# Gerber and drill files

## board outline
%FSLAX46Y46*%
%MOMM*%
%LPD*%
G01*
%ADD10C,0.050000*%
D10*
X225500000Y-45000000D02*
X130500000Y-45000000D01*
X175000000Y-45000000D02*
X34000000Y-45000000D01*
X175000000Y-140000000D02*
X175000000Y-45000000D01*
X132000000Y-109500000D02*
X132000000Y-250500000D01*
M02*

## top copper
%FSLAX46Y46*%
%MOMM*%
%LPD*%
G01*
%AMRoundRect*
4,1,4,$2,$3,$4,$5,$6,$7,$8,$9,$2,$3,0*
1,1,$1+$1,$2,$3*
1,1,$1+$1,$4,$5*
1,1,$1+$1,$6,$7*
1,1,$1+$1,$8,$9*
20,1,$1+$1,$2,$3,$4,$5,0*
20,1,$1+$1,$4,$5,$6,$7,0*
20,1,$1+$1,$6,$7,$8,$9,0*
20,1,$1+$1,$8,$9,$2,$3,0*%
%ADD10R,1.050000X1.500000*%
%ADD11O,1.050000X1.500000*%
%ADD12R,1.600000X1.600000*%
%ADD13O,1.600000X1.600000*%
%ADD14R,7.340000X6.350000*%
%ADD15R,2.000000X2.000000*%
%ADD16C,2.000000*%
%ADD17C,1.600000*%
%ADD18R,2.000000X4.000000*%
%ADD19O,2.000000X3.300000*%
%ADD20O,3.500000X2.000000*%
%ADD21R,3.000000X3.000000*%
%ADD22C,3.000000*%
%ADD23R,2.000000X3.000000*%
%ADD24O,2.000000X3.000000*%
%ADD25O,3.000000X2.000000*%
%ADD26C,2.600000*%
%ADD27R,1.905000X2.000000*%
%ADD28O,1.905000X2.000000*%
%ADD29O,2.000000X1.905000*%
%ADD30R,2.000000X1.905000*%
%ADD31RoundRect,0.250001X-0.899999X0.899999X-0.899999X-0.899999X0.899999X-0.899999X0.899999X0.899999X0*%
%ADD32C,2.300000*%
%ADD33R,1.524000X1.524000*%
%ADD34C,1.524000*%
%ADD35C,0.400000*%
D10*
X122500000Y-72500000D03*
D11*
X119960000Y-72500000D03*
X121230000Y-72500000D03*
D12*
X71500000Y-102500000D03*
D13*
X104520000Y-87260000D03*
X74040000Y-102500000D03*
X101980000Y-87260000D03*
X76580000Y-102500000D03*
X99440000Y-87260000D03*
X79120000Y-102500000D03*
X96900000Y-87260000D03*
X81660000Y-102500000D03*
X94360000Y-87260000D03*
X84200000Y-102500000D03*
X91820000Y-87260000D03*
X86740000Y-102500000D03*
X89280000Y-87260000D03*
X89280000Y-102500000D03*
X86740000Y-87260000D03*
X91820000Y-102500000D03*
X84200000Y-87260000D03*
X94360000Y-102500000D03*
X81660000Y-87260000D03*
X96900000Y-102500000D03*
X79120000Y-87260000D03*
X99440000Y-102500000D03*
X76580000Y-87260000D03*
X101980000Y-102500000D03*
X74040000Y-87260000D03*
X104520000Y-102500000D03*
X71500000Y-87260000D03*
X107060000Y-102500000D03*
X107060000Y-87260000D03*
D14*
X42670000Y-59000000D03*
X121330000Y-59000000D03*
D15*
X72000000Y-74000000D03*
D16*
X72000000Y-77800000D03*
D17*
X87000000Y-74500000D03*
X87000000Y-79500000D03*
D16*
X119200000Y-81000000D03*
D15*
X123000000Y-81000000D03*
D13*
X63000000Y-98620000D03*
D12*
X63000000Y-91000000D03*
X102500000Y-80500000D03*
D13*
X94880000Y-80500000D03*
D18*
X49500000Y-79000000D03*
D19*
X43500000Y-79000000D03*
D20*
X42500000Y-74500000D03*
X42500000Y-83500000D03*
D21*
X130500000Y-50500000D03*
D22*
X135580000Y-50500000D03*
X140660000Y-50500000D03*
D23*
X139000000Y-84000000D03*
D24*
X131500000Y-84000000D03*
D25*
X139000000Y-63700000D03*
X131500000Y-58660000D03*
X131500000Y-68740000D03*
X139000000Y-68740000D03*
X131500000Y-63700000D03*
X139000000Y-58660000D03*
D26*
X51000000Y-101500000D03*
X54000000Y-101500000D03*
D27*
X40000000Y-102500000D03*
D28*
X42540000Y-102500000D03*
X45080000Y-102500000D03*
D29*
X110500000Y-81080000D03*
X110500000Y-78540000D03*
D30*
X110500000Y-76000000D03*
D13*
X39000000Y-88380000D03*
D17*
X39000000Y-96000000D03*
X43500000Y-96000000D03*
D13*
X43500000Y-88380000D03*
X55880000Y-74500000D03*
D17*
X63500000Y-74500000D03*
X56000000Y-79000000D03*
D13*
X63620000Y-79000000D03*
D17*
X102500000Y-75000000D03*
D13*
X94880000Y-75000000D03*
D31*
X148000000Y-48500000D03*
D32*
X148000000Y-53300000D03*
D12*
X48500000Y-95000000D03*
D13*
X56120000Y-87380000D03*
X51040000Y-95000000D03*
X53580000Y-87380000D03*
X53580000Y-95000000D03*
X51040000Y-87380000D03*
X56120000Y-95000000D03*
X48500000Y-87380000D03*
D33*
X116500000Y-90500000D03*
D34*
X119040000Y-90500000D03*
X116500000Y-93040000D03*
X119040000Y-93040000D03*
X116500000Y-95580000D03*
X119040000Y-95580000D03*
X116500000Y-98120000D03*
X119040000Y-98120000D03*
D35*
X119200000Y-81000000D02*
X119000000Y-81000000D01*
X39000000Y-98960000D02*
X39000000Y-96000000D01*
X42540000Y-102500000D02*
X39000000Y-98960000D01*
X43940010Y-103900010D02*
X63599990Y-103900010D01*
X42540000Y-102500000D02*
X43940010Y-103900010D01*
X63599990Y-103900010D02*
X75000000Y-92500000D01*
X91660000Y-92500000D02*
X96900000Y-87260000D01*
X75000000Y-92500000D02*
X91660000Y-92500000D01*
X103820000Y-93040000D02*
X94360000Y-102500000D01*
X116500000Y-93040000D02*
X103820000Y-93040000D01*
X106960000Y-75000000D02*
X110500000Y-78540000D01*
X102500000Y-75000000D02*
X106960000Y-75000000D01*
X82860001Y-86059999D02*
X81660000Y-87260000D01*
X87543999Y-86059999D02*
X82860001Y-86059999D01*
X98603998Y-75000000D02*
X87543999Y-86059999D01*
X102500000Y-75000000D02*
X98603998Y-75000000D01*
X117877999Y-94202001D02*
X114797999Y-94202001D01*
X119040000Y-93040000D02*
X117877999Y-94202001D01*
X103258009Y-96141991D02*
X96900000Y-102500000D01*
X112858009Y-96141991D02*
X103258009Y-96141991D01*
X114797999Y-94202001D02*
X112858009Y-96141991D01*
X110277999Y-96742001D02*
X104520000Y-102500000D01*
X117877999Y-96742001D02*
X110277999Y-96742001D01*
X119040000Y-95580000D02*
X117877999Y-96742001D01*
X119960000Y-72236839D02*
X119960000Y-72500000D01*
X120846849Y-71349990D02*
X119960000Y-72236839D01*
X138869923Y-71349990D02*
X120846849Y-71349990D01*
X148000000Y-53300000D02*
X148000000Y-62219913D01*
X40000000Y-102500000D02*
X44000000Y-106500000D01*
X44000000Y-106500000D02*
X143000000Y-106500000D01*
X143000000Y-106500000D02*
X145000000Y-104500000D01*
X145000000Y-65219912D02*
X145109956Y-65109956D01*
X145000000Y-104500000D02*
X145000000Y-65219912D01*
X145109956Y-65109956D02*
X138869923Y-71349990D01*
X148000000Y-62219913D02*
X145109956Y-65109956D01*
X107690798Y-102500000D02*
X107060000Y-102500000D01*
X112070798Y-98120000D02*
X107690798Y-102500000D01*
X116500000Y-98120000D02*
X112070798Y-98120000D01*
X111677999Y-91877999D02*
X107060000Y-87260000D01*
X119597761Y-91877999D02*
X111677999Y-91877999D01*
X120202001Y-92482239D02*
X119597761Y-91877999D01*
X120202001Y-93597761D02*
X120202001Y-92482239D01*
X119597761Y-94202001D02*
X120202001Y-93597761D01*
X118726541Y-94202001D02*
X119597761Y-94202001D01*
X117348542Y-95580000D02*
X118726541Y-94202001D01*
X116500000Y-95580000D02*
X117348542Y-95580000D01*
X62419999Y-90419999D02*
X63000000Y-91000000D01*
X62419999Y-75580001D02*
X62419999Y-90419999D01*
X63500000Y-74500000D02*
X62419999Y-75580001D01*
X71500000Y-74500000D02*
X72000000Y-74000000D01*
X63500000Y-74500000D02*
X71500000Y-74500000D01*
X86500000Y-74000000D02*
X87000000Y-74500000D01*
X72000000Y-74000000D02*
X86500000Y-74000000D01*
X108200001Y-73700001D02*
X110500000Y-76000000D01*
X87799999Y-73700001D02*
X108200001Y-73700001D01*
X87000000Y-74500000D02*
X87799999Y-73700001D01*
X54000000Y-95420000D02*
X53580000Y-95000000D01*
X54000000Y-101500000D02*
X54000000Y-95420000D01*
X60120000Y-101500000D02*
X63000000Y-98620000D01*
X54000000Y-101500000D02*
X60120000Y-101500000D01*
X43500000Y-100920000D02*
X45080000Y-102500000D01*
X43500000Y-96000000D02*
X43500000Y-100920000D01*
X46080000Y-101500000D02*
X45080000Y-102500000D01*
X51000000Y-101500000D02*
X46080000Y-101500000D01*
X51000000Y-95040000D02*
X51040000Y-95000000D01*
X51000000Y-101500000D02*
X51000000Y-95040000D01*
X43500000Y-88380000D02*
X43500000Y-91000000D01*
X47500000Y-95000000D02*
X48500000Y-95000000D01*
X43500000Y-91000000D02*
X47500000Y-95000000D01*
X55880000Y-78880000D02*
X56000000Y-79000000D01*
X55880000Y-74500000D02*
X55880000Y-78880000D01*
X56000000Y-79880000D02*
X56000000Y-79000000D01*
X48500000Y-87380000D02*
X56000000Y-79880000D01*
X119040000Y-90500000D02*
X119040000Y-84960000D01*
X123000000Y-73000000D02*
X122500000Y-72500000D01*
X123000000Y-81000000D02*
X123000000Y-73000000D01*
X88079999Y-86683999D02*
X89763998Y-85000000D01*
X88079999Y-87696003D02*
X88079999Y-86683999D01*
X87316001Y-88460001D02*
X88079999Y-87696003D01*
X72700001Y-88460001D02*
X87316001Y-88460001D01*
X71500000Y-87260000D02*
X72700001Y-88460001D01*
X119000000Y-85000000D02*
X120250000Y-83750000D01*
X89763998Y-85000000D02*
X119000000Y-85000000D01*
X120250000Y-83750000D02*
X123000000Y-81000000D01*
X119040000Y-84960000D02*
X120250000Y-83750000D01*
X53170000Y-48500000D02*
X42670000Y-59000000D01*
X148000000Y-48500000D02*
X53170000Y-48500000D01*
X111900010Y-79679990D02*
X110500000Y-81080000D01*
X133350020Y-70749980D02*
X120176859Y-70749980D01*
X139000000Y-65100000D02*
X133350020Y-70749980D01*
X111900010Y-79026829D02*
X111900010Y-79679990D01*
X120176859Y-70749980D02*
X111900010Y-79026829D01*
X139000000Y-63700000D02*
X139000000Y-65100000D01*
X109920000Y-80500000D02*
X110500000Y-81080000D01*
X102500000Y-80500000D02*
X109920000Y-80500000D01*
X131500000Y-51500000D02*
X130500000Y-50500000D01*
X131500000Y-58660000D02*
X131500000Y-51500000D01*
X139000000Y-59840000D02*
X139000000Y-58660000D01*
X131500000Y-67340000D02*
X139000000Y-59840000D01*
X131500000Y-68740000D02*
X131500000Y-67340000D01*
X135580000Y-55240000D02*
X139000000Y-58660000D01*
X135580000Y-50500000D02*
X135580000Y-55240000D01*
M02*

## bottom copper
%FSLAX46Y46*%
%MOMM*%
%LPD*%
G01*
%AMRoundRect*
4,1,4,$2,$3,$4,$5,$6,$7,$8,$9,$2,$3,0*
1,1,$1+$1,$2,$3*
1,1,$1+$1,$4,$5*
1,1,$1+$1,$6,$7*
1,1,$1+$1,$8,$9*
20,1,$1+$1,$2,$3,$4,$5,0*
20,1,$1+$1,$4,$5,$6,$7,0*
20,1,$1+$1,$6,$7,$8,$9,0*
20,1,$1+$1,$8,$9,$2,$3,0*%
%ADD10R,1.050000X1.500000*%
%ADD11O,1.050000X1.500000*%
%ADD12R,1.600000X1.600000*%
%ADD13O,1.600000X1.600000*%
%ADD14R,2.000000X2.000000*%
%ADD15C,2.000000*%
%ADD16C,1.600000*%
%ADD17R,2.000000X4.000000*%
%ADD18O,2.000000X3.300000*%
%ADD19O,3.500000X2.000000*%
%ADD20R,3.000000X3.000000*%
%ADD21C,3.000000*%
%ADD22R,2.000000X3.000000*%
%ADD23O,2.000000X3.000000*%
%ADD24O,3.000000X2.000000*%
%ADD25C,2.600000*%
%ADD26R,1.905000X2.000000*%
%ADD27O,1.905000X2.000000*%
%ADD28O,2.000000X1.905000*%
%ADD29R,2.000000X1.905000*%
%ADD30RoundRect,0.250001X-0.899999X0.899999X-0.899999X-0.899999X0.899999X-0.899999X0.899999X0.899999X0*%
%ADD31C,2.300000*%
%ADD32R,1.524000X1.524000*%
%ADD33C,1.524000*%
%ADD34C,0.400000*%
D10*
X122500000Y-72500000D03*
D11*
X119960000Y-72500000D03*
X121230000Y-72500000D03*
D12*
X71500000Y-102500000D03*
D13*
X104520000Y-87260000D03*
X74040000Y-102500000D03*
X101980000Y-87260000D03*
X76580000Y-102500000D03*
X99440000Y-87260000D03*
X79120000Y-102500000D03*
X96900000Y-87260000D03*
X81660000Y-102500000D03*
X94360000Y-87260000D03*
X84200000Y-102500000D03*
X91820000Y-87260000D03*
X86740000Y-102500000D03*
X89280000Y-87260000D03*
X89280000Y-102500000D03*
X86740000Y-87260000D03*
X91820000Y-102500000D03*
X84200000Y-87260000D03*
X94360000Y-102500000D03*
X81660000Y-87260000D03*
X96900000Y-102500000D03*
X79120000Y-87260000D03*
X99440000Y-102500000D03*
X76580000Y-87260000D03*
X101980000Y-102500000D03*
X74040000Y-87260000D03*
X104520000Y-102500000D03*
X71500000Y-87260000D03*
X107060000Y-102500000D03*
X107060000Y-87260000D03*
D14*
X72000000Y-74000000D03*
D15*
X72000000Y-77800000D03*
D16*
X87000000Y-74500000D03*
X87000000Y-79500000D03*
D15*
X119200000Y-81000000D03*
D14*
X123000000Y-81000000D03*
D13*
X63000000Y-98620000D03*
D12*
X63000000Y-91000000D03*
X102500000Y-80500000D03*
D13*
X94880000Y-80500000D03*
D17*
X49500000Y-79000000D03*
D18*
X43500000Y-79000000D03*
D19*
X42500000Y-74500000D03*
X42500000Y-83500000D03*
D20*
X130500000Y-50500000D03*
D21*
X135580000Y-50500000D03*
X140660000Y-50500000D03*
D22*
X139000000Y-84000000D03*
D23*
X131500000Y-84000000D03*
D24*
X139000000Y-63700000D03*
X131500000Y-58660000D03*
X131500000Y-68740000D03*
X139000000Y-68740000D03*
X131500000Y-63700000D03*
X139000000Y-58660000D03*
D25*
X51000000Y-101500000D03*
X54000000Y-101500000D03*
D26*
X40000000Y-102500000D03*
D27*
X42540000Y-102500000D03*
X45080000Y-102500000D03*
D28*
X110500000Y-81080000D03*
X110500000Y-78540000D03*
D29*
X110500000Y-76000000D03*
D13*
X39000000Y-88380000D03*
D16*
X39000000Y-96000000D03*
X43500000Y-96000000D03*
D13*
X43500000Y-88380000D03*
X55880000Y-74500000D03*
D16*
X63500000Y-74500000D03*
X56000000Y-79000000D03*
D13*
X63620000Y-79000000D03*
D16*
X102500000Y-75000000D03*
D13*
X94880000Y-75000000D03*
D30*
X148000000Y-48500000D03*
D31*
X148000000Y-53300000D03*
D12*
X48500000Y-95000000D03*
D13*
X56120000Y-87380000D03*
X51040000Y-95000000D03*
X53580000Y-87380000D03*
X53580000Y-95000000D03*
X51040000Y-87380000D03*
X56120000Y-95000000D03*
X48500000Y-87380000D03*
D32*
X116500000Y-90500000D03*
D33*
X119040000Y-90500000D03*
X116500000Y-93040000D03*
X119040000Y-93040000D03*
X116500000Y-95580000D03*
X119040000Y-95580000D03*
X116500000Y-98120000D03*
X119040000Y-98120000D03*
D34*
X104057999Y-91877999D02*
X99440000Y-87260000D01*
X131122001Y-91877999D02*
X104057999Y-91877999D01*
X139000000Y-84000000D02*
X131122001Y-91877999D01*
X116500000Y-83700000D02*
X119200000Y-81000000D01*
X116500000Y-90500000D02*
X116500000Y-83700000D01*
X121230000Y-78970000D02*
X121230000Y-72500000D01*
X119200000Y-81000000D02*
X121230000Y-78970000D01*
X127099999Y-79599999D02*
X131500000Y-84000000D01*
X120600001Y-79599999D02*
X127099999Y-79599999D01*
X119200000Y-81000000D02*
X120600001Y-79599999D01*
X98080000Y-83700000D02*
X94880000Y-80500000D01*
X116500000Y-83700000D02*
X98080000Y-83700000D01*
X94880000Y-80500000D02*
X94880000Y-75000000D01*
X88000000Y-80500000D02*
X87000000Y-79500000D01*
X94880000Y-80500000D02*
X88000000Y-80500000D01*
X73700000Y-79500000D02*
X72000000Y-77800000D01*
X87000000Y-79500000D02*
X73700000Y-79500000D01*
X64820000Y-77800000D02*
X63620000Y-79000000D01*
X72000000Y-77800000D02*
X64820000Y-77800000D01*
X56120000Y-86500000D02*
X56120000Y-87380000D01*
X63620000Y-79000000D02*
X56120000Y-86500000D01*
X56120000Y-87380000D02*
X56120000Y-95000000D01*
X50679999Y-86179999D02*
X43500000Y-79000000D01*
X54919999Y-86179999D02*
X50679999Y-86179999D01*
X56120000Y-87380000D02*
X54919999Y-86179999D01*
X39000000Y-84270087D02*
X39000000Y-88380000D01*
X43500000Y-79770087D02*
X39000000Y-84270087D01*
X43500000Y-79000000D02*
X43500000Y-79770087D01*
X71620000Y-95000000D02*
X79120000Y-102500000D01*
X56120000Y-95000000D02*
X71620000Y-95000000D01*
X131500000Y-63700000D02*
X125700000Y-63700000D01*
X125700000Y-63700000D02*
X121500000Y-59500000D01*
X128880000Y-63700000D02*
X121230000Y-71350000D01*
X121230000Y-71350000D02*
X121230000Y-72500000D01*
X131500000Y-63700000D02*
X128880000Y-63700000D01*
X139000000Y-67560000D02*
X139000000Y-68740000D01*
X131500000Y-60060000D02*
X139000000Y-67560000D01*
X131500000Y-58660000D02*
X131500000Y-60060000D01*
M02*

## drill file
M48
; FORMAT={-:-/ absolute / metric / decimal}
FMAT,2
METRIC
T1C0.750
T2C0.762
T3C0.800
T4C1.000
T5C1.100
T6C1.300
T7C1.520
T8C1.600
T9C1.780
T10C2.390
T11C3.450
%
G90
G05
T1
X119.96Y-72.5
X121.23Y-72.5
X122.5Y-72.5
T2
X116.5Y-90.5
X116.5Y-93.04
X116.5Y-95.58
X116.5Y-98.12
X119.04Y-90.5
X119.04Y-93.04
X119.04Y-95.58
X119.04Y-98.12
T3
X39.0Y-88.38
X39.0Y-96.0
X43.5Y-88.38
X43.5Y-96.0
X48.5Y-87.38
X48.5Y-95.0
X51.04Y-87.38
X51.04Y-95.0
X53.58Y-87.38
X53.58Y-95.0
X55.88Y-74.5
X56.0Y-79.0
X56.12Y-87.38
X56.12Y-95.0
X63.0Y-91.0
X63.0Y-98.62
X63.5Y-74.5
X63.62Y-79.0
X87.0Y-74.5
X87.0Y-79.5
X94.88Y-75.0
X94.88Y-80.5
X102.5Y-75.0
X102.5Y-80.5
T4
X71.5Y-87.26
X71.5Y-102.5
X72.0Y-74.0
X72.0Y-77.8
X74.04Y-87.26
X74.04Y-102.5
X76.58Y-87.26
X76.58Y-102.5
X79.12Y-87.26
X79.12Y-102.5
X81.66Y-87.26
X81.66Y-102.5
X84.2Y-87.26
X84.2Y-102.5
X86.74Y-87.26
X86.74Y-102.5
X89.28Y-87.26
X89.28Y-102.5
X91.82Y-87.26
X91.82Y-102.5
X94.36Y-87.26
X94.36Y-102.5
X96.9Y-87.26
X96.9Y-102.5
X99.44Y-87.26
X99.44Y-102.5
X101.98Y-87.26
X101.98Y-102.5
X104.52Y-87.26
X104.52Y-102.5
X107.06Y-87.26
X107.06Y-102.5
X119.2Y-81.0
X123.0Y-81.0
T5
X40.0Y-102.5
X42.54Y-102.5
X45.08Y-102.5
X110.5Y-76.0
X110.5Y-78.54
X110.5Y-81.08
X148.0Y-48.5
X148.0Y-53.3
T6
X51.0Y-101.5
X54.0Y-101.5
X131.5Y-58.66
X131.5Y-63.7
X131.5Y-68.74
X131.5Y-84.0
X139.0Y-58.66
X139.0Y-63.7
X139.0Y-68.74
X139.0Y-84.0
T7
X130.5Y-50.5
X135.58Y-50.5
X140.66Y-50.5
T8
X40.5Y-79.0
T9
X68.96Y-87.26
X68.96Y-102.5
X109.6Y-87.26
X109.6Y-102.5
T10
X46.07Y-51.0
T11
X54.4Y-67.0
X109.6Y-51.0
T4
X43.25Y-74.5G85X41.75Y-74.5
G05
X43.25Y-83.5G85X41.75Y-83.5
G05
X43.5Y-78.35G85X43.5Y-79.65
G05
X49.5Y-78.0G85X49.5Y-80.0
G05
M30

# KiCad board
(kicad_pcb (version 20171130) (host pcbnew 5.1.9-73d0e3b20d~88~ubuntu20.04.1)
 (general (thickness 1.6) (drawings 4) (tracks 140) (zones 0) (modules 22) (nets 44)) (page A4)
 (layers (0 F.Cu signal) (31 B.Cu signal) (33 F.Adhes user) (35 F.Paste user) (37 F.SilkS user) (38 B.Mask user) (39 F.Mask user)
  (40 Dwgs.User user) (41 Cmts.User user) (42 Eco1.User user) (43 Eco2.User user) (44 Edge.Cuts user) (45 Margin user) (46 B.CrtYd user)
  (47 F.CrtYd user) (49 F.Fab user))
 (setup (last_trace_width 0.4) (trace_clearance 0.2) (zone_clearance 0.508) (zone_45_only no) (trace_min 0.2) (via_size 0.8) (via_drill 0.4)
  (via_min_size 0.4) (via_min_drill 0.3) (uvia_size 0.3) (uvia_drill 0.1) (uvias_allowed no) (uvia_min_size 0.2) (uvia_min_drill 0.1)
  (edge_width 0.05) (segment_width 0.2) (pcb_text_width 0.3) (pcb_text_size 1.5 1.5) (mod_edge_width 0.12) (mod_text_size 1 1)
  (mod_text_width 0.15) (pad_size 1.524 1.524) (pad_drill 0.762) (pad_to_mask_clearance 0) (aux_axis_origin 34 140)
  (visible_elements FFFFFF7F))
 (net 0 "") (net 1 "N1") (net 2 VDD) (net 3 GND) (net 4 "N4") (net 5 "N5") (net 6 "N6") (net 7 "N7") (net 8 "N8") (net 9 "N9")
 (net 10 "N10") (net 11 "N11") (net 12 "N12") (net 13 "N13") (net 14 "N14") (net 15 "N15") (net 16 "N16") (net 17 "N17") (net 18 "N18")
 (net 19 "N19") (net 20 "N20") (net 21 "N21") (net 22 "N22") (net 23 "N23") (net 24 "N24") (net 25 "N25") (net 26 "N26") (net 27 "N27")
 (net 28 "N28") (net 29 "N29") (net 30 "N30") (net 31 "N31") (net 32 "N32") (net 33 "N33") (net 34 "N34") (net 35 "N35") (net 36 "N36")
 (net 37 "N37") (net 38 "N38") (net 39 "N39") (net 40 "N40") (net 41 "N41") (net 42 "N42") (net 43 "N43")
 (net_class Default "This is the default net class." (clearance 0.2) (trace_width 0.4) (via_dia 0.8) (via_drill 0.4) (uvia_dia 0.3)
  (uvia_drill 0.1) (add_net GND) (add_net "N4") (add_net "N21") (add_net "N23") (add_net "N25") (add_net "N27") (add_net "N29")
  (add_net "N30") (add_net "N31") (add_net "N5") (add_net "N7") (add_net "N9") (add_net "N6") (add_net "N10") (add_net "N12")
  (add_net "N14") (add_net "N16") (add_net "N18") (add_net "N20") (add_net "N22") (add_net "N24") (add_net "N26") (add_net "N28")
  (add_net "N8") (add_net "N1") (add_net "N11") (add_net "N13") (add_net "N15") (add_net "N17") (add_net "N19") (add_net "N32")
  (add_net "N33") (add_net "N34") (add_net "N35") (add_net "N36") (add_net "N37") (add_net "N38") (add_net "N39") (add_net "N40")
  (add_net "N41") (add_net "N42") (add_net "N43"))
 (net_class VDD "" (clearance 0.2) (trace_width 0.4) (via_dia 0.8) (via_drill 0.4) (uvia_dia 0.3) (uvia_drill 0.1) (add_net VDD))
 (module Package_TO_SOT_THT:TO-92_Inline (layer F.Cu) (at 122.5 72.5 180)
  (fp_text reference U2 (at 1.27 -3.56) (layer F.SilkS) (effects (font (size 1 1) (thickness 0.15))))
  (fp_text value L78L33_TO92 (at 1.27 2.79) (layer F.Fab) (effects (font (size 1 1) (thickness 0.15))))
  (pad 1 thru_hole rect (at 0 0 180) (size 1.05 1.5) (drill 0.75) (layers *.Cu *.Mask) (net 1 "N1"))
  (pad 3 thru_hole oval (at 2.54 0 180) (size 1.05 1.5) (drill 0.75) (layers *.Cu *.Mask) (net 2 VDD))
  (pad 2 thru_hole oval (at 1.27 0 180) (size 1.05 1.5) (drill 0.75) (layers *.Cu *.Mask) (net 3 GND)))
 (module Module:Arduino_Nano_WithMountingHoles (layer F.Cu) (at 71.5 102.5 90)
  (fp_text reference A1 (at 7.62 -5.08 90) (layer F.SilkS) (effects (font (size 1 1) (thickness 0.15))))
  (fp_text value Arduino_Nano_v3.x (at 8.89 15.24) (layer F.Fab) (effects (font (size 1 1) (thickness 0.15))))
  (pad 1 thru_hole rect (at 0 0 90) (size 1.6 1.6) (drill 1) (layers *.Cu *.Mask) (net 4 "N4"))
  (pad 17 thru_hole oval (at 15.24 33.02 90) (size 1.6 1.6) (drill 1) (layers *.Cu *.Mask) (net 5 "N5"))
  (pad 2 thru_hole oval (at 0 2.54 90) (size 1.6 1.6) (drill 1) (layers *.Cu *.Mask) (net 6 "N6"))
  (pad 18 thru_hole oval (at 15.24 30.48 90) (size 1.6 1.6) (drill 1) (layers *.Cu *.Mask) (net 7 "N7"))
  (pad 3 thru_hole oval (at 0 5.08 90) (size 1.6 1.6) (drill 1) (layers *.Cu *.Mask) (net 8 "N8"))
  (pad 19 thru_hole oval (at 15.24 27.94 90) (size 1.6 1.6) (drill 1) (layers *.Cu *.Mask) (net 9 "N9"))
  (pad 4 thru_hole oval (at 0 7.62 90) (size 1.6 1.6) (drill 1) (layers *.Cu *.Mask) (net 3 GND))
  (pad 20 thru_hole oval (at 15.24 25.4 90) (size 1.6 1.6) (drill 1) (layers *.Cu *.Mask) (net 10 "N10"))
  (pad 5 thru_hole oval (at 0 10.16 90) (size 1.6 1.6) (drill 1) (layers *.Cu *.Mask) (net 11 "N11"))
  (pad 21 thru_hole oval (at 15.24 22.86 90) (size 1.6 1.6) (drill 1) (layers *.Cu *.Mask) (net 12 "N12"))
  (pad 6 thru_hole oval (at 0 12.7 90) (size 1.6 1.6) (drill 1) (layers *.Cu *.Mask) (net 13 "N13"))
  (pad 22 thru_hole oval (at 15.24 20.32 90) (size 1.6 1.6) (drill 1) (layers *.Cu *.Mask) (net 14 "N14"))
  (pad 7 thru_hole oval (at 0 15.24 90) (size 1.6 1.6) (drill 1) (layers *.Cu *.Mask) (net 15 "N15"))
  (pad 23 thru_hole oval (at 15.24 17.78 90) (size 1.6 1.6) (drill 1) (layers *.Cu *.Mask) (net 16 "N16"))
  (pad 8 thru_hole oval (at 0 17.78 90) (size 1.6 1.6) (drill 1) (layers *.Cu *.Mask) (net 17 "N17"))
  (pad 24 thru_hole oval (at 15.24 15.24 90) (size 1.6 1.6) (drill 1) (layers *.Cu *.Mask) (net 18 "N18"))
  (pad 9 thru_hole oval (at 0 20.32 90) (size 1.6 1.6) (drill 1) (layers *.Cu *.Mask) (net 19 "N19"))
  (pad 25 thru_hole oval (at 15.24 12.7 90) (size 1.6 1.6) (drill 1) (layers *.Cu *.Mask) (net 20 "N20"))
  (pad 10 thru_hole oval (at 0 22.86 90) (size 1.6 1.6) (drill 1) (layers *.Cu *.Mask) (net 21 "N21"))
  (pad 26 thru_hole oval (at 15.24 10.16 90) (size 1.6 1.6) (drill 1) (layers *.Cu *.Mask) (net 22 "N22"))
  (pad 11 thru_hole oval (at 0 25.4 90) (size 1.6 1.6) (drill 1) (layers *.Cu *.Mask) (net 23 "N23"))
  (pad 27 thru_hole oval (at 15.24 7.62 90) (size 1.6 1.6) (drill 1) (layers *.Cu *.Mask) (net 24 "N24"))
  (pad 12 thru_hole oval (at 0 27.94 90) (size 1.6 1.6) (drill 1) (layers *.Cu *.Mask) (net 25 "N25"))
  (pad 28 thru_hole oval (at 15.24 5.08 90) (size 1.6 1.6) (drill 1) (layers *.Cu *.Mask) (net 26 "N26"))
  (pad 13 thru_hole oval (at 0 30.48 90) (size 1.6 1.6) (drill 1) (layers *.Cu *.Mask) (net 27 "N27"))
  (pad 29 thru_hole oval (at 15.24 2.54 90) (size 1.6 1.6) (drill 1) (layers *.Cu *.Mask) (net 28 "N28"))
  (pad 14 thru_hole oval (at 0 33.02 90) (size 1.6 1.6) (drill 1) (layers *.Cu *.Mask) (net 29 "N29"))
  (pad 30 thru_hole oval (at 15.24 0 90) (size 1.6 1.6) (drill 1) (layers *.Cu *.Mask) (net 1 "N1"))
  (pad 15 thru_hole oval (at 0 35.56 90) (size 1.6 1.6) (drill 1) (layers *.Cu *.Mask) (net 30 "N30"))
  (pad 16 thru_hole oval (at 15.24 35.56 90) (size 1.6 1.6) (drill 1) (layers *.Cu *.Mask) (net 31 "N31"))
  (pad "" np_thru_hole circle (at 0 -2.54 90) (size 1.78 1.78) (drill 1.78) (layers *.Cu *.Mask))
  (pad "" np_thru_hole circle (at 15.24 -2.54 90) (size 1.78 1.78) (drill 1.78) (layers *.Cu *.Mask))
  (pad "" np_thru_hole circle (at 15.24 38.1 90) (size 1.78 1.78) (drill 1.78) (layers *.Cu *.Mask))
  (pad "" np_thru_hole circle (at 0 38.1 90) (size 1.78 1.78) (drill 1.78) (layers *.Cu *.Mask)))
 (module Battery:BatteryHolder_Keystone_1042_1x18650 (layer F.Cu) (at 82 59)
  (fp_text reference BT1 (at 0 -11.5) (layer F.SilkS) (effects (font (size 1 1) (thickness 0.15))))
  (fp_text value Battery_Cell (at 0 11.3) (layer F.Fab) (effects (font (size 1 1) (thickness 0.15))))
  (pad 1 smd rect (at -39.33 0) (size 7.34 6.35) (layers F.Cu F.Paste F.Mask) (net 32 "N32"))
  (pad 2 smd rect (at 39.33 0) (size 7.34 6.35) (layers F.Cu F.Paste F.Mask) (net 3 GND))
  (pad "" np_thru_hole circle (at 27.6 -8) (size 3.45 3.45) (drill 3.45) (layers *.Cu *.Mask))
  (pad "" np_thru_hole circle (at -27.6 8) (size 3.45 3.45) (drill 3.45) (layers *.Cu *.Mask))
  (pad "" np_thru_hole circle (at -35.93 -8) (size 2.39 2.39) (drill 2.39) (layers *.Cu *.Mask)))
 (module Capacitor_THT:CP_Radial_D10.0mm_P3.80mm (layer F.Cu) (at 72 74 270)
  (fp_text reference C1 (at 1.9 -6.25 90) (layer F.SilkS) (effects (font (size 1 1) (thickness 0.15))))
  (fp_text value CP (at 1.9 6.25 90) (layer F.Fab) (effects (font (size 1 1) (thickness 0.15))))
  (pad 1 thru_hole rect (at 0 0 270) (size 2 2) (drill 1) (layers *.Cu *.Mask) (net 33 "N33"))
  (pad 2 thru_hole circle (at 3.8 0 270) (size 2 2) (drill 1) (layers *.Cu *.Mask) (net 3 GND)))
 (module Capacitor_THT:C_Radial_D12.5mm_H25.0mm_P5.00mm (layer F.Cu) (at 87 74.5 270)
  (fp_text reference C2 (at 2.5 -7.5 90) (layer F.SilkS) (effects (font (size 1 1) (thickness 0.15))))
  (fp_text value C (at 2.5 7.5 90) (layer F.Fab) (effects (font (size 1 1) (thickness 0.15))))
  (pad 1 thru_hole circle (at 0 0 270) (size 1.6 1.6) (drill 0.8) (layers *.Cu *.Mask) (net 33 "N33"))
  (pad 2 thru_hole circle (at 5 0 270) (size 1.6 1.6) (drill 0.8) (layers *.Cu *.Mask) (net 3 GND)))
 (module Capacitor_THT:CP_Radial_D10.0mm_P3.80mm (layer F.Cu) (at 123 81 180)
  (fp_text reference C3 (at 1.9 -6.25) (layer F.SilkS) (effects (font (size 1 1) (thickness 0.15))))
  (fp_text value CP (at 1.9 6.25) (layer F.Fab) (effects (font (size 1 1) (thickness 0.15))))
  (pad 2 thru_hole circle (at 3.8 0 180) (size 2 2) (drill 1) (layers *.Cu *.Mask) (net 3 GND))
  (pad 1 thru_hole rect (at 0 0 180) (size 2 2) (drill 1) (layers *.Cu *.Mask) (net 1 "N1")))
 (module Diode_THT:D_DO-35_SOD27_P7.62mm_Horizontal (layer F.Cu) (at 63 91 270)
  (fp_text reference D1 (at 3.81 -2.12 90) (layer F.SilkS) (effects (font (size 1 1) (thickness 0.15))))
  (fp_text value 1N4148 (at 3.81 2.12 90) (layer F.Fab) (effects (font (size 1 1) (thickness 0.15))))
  (pad 2 thru_hole oval (at 7.62 0 270) (size 1.6 1.6) (drill 0.8) (layers *.Cu *.Mask) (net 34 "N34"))
  (pad 1 thru_hole rect (at 0 0 270) (size 1.6 1.6) (drill 0.8) (layers *.Cu *.Mask) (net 33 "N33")))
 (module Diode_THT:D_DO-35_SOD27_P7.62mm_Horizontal (layer F.Cu) (at 102.5 80.5 180)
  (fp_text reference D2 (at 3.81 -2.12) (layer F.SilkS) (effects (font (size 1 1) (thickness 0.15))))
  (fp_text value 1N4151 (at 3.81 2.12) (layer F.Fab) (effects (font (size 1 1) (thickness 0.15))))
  (pad 1 thru_hole rect (at 0 0 180) (size 1.6 1.6) (drill 0.8) (layers *.Cu *.Mask) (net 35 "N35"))
  (pad 2 thru_hole oval (at 7.62 0 180) (size 1.6 1.6) (drill 0.8) (layers *.Cu *.Mask) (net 3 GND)))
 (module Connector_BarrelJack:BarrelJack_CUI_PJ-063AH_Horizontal (layer F.Cu) (at 49.5 79 270)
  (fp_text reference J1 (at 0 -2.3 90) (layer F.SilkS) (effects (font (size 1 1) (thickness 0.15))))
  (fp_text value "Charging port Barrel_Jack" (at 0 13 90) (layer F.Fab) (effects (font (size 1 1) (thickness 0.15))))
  (pad 1 thru_hole rect (at 0 0 270) (size 4 2) (drill oval 3 1) (layers *.Cu *.Mask) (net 32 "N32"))
  (pad 2 thru_hole oval (at 0 6 270) (size 3.3 2) (drill oval 2.3 1) (layers *.Cu *.Mask) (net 3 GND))
  (pad MP thru_hole oval (at -4.5 7 270) (size 2 3.5) (drill oval 1 2.5) (layers *.Cu *.Mask))
  (pad MP thru_hole oval (at 4.5 7 270) (size 2 3.5) (drill oval 1 2.5) (layers *.Cu *.Mask))
  (pad "" np_thru_hole circle (at 0 9 270) (size 1.6 1.6) (drill 1.6) (layers *.Cu *.Mask)))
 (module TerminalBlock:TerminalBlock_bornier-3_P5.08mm (layer F.Cu) (at 130.5 50.5)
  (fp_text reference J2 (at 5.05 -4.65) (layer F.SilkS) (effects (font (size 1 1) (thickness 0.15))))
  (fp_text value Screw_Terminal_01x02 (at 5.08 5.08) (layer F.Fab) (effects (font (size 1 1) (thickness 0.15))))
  (pad 1 thru_hole rect (at 0 0) (size 3 3) (drill 1.52) (layers *.Cu *.Mask) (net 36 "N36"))
  (pad 2 thru_hole circle (at 5.08 0) (size 3 3) (drill 1.52) (layers *.Cu *.Mask) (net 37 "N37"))
  (pad 3 thru_hole circle (at 10.16 0) (size 3 3) (drill 1.52) (layers *.Cu *.Mask)))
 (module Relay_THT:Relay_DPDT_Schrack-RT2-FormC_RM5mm (layer F.Cu) (at 139 84 90)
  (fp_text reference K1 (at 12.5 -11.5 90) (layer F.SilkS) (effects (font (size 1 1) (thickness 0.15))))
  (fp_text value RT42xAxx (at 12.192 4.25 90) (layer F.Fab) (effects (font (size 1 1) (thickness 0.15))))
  (pad A1 thru_hole rect (at 0 0 270) (size 3 2) (drill 1.3) (layers *.Cu *.Mask) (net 9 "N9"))
  (pad A2 thru_hole oval (at 0 -7.5 270) (size 3 2) (drill 1.3) (layers *.Cu *.Mask) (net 3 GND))
  (pad 11 thru_hole oval (at 20.3 0 270) (size 2 3) (drill 1.3) (layers *.Cu *.Mask) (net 35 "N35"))
  (pad 24 thru_hole oval (at 25.34 -7.5 270) (size 2 3) (drill 1.3) (layers *.Cu *.Mask) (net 36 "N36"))
  (pad 22 thru_hole oval (at 15.26 -7.5 270) (size 2 3) (drill 1.3) (layers *.Cu *.Mask) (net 37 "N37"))
  (pad 12 thru_hole oval (at 15.26 0 270) (size 2 3) (drill 1.3) (layers *.Cu *.Mask) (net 36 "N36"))
  (pad 21 thru_hole oval (at 20.3 -7.5 270) (size 2 3) (drill 1.3) (layers *.Cu *.Mask) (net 3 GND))
  (pad 14 thru_hole oval (at 25.34 0 270) (size 2 3) (drill 1.3) (layers *.Cu *.Mask) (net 37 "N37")))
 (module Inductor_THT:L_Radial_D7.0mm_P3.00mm (layer F.Cu) (at 51 101.5)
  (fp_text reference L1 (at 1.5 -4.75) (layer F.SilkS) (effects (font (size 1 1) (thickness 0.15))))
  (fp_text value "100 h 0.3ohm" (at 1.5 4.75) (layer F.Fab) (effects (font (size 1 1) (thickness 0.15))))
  (pad 1 thru_hole circle (at 0 0) (size 2.6 2.6) (drill 1.3) (layers *.Cu *.Mask) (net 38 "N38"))
  (pad 2 thru_hole circle (at 3 0) (size 2.6 2.6) (drill 1.3) (layers *.Cu *.Mask) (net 34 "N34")))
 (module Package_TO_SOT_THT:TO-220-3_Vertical (layer F.Cu) (at 40 102.5)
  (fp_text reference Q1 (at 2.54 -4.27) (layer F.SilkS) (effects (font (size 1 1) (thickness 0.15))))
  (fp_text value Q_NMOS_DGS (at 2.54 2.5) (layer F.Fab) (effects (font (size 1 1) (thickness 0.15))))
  (pad 1 thru_hole rect (at 0 0) (size 1.905 2) (drill 1.1) (layers *.Cu *.Mask) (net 2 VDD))
  (pad 2 thru_hole oval (at 2.54 0) (size 1.905 2) (drill 1.1) (layers *.Cu *.Mask) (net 10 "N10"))
  (pad 3 thru_hole oval (at 5.08 0) (size 1.905 2) (drill 1.1) (layers *.Cu *.Mask) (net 38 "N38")))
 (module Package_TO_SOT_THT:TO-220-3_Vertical (layer F.Cu) (at 110.5 76 270)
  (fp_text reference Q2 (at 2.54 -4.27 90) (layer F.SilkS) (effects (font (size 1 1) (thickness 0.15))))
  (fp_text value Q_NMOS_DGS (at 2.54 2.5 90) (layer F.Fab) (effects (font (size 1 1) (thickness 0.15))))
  (pad 3 thru_hole oval (at 5.08 0 270) (size 1.905 2) (drill 1.1) (layers *.Cu *.Mask) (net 35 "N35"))
  (pad 2 thru_hole oval (at 2.54 0 270) (size 1.905 2) (drill 1.1) (layers *.Cu *.Mask) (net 22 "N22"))
  (pad 1 thru_hole rect (at 0 0 270) (size 1.905 2) (drill 1.1) (layers *.Cu *.Mask) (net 33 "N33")))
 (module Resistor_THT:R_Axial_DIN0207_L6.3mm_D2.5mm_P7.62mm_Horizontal (layer F.Cu) (at 39 96 90)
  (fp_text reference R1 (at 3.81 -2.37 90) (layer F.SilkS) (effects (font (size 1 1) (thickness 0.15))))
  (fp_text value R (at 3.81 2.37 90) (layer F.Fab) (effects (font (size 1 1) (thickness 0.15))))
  (pad 2 thru_hole oval (at 7.62 0 90) (size 1.6 1.6) (drill 0.8) (layers *.Cu *.Mask) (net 3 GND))
  (pad 1 thru_hole circle (at 0 0 90) (size 1.6 1.6) (drill 0.8) (layers *.Cu *.Mask) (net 10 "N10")))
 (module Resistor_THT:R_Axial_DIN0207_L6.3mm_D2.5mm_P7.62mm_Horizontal (layer F.Cu) (at 43.5 96 90)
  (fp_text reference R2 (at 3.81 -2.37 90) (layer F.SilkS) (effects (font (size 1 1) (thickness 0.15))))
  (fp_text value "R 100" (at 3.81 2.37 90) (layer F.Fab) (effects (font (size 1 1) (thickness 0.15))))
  (pad 1 thru_hole circle (at 0 0 90) (size 1.6 1.6) (drill 0.8) (layers *.Cu *.Mask) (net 38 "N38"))
  (pad 2 thru_hole oval (at 7.62 0 90) (size 1.6 1.6) (drill 0.8) (layers *.Cu *.Mask) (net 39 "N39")))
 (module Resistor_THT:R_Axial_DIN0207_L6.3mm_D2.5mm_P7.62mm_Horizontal (layer F.Cu) (at 63.5 74.5 180)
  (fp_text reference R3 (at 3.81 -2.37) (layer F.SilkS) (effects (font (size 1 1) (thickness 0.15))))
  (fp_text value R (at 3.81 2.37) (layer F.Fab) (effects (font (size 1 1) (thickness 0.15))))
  (pad 2 thru_hole oval (at 7.62 0 180) (size 1.6 1.6) (drill 0.8) (layers *.Cu *.Mask) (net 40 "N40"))
  (pad 1 thru_hole circle (at 0 0 180) (size 1.6 1.6) (drill 0.8) (layers *.Cu *.Mask) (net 33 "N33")))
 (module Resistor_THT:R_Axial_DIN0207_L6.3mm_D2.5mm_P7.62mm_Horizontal (layer F.Cu) (at 56 79)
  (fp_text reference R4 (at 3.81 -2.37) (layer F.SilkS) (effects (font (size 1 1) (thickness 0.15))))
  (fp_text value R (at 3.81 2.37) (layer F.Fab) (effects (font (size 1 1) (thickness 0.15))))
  (pad 1 thru_hole circle (at 0 0) (size 1.6 1.6) (drill 0.8) (layers *.Cu *.Mask) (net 40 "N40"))
  (pad 2 thru_hole oval (at 7.62 0) (size 1.6 1.6) (drill 0.8) (layers *.Cu *.Mask) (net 3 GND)))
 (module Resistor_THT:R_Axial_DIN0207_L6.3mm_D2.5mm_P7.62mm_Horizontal (layer F.Cu) (at 102.5 75 180)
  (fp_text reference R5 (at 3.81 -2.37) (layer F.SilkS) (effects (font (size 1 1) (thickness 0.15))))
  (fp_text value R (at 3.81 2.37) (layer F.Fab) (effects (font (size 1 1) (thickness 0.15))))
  (pad 1 thru_hole circle (at 0 0 180) (size 1.6 1.6) (drill 0.8) (layers *.Cu *.Mask) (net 22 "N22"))
  (pad 2 thru_hole oval (at 7.62 0 180) (size 1.6 1.6) (drill 0.8) (layers *.Cu *.Mask) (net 3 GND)))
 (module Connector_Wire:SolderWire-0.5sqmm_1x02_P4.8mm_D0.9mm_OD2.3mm (layer F.Cu) (at 148 48.5 270)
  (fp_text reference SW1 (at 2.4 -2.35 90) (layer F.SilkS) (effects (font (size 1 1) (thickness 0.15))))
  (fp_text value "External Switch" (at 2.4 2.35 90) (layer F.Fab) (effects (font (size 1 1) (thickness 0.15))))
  (pad 1 thru_hole roundrect (at 0 0 270) (size 2.3 2.3) (drill 1.1) (layers *.Cu *.Mask) (roundrect_rratio 0.108696) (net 32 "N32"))
  (pad 2 thru_hole circle (at 4.8 0 270) (size 2.3 2.3) (drill 1.1) (layers *.Cu *.Mask) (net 2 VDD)))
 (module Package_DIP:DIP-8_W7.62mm (layer F.Cu) (at 48.5 95 90)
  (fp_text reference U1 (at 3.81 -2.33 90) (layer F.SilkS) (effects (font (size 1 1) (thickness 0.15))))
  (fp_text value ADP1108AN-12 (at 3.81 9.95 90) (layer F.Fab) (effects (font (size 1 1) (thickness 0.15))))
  (pad 1 thru_hole rect (at 0 0 90) (size 1.6 1.6) (drill 0.8) (layers *.Cu *.Mask) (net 39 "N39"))
  (pad 5 thru_hole oval (at 7.62 7.62 90) (size 1.6 1.6) (drill 0.8) (layers *.Cu *.Mask) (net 3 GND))
  (pad 2 thru_hole oval (at 0 2.54 90) (size 1.6 1.6) (drill 0.8) (layers *.Cu *.Mask) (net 38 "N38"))
  (pad 6 thru_hole oval (at 7.62 5.08 90) (size 1.6 1.6) (drill 0.8) (layers *.Cu *.Mask) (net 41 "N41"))
  (pad 3 thru_hole oval (at 0 5.08 90) (size 1.6 1.6) (drill 0.8) (layers *.Cu *.Mask) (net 34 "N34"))
  (pad 7 thru_hole oval (at 7.62 2.54 90) (size 1.6 1.6) (drill 0.8) (layers *.Cu *.Mask) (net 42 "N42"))
  (pad 4 thru_hole oval (at 0 7.62 90) (size 1.6 1.6) (drill 0.8) (layers *.Cu *.Mask) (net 3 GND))
  (pad 8 thru_hole oval (at 7.62 0 90) (size 1.6 1.6) (drill 0.8) (layers *.Cu *.Mask) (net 40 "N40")))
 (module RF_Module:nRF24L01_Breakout (layer F.Cu) (at 116.5 90.5)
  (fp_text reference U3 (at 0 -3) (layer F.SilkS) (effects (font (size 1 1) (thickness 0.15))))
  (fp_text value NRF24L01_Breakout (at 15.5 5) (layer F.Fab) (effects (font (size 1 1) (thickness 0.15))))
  (pad 1 thru_hole rect (at 0 0) (size 1.524 1.524) (drill 0.762) (layers *.Cu *.Mask) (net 3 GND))
  (pad 2 thru_hole circle (at 2.54 0) (size 1.524 1.524) (drill 0.762) (layers *.Cu *.Mask) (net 1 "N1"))
  (pad 3 thru_hole circle (at 0 2.54) (size 1.524 1.524) (drill 0.762) (layers *.Cu *.Mask) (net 21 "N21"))
  (pad 4 thru_hole circle (at 2.54 2.54) (size 1.524 1.524) (drill 0.762) (layers *.Cu *.Mask) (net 23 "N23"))
  (pad 5 thru_hole circle (at 0 5.08) (size 1.524 1.524) (drill 0.762) (layers *.Cu *.Mask) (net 31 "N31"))
  (pad 6 thru_hole circle (at 2.54 5.08) (size 1.524 1.524) (drill 0.762) (layers *.Cu *.Mask) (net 29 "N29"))
  (pad 7 thru_hole circle (at 0 7.62) (size 1.524 1.524) (drill 0.762) (layers *.Cu *.Mask) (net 30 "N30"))
  (pad 8 thru_hole circle (at 2.54 7.62) (size 1.524 1.524) (drill 0.762) (layers *.Cu *.Mask) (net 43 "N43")))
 (gr_line (start 225.5 45) (end 130.5 45) (layer Edge.Cuts) (width 0.05))
 (gr_line (start 175 45) (end 34 45) (layer Edge.Cuts) (width 0.05))
 (gr_line (start 175 140) (end 175 45) (layer Edge.Cuts) (width 0.05))
 (gr_line (start 132 109.5) (end 132 250.5) (layer Edge.Cuts) (width 0.05))
 (segment (start 104.057999 91.877999) (end 99.44 87.26) (width 0.4) (layer B.Cu) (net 9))
 (segment (start 131.122001 91.877999) (end 104.057999 91.877999) (width 0.4) (layer B.Cu) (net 9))
 (segment (start 139 84) (end 131.122001 91.877999) (width 0.4) (layer B.Cu) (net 9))
 (segment (start 116.5 83.7) (end 119.2 81) (width 0.4) (layer B.Cu) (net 3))
 (segment (start 116.5 90.5) (end 116.5 83.7) (width 0.4) (layer B.Cu) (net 3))
 (segment (start 119.2 81) (end 119 81) (width 0.4) (layer F.Cu) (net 3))
 (segment (start 121.23 78.97) (end 121.23 72.5) (width 0.4) (layer B.Cu) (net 3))
 (segment (start 119.2 81) (end 121.23 78.97) (width 0.4) (layer B.Cu) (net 3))
 (segment (start 127.099999 79.599999) (end 131.5 84) (width 0.4) (layer B.Cu) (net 3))
 (segment (start 120.600001 79.599999) (end 127.099999 79.599999) (width 0.4) (layer B.Cu) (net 3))
 (segment (start 119.2 81) (end 120.600001 79.599999) (width 0.4) (layer B.Cu) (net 3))
 (segment (start 98.08 83.7) (end 94.88 80.5) (width 0.4) (layer B.Cu) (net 3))
 (segment (start 116.5 83.7) (end 98.08 83.7) (width 0.4) (layer B.Cu) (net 3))
 (segment (start 94.88 80.5) (end 94.88 75) (width 0.4) (layer B.Cu) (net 3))
 (segment (start 88 80.5) (end 87 79.5) (width 0.4) (layer B.Cu) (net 3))
 (segment (start 94.88 80.5) (end 88 80.5) (width 0.4) (layer B.Cu) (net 3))
 (segment (start 73.7 79.5) (end 72 77.8) (width 0.4) (layer B.Cu) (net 3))
 (segment (start 87 79.5) (end 73.7 79.5) (width 0.4) (layer B.Cu) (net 3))
 (segment (start 64.82 77.8) (end 63.62 79) (width 0.4) (layer B.Cu) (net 3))
 (segment (start 72 77.8) (end 64.82 77.8) (width 0.4) (layer B.Cu) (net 3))
 (segment (start 56.12 86.5) (end 56.12 87.38) (width 0.4) (layer B.Cu) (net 3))
 (segment (start 63.62 79) (end 56.12 86.5) (width 0.4) (layer B.Cu) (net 3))
 (segment (start 56.12 87.38) (end 56.12 95) (width 0.4) (layer B.Cu) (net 3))
 (segment (start 50.679999 86.179999) (end 43.5 79) (width 0.4) (layer B.Cu) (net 3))
 (segment (start 54.919999 86.179999) (end 50.679999 86.179999) (width 0.4) (layer B.Cu) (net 3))
 (segment (start 56.12 87.38) (end 54.919999 86.179999) (width 0.4) (layer B.Cu) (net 3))
 (segment (start 39 84.270087) (end 39 88.38) (width 0.4) (layer B.Cu) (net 3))
 (segment (start 43.5 79.770087) (end 39 84.270087) (width 0.4) (layer B.Cu) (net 3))
 (segment (start 43.5 79) (end 43.5 79.770087) (width 0.4) (layer B.Cu) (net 3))
 (segment (start 71.62 95) (end 79.12 102.5) (width 0.4) (layer B.Cu) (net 3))
 (segment (start 56.12 95) (end 71.62 95) (width 0.4) (layer B.Cu) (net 3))
 (segment (start 131.5 63.7) (end 125.7 63.7) (width 0.4) (layer B.Cu) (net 3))
 (segment (start 125.7 63.7) (end 121.5 59.5) (width 0.4) (layer B.Cu) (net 3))
 (segment (start 128.88 63.7) (end 121.23 71.35) (width 0.4) (layer B.Cu) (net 3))
 (segment (start 121.23 71.35) (end 121.23 72.5) (width 0.4) (layer B.Cu) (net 3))
 (segment (start 131.5 63.7) (end 128.88 63.7) (width 0.4) (layer B.Cu) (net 3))
 (segment (start 39 98.96) (end 39 96) (width 0.4) (layer F.Cu) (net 10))
 (segment (start 42.54 102.5) (end 39 98.96) (width 0.4) (layer F.Cu) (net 10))
 (segment (start 43.94001 103.90001) (end 63.59999 103.90001) (width 0.4) (layer F.Cu) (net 10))
 (segment (start 42.54 102.5) (end 43.94001 103.90001) (width 0.4) (layer F.Cu) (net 10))
 (segment (start 63.59999 103.90001) (end 75 92.5) (width 0.4) (layer F.Cu) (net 10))
 (segment (start 91.66 92.5) (end 96.9 87.26) (width 0.4) (layer F.Cu) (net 10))
 (segment (start 75 92.5) (end 91.66 92.5) (width 0.4) (layer F.Cu) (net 10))
 (segment (start 103.82 93.04) (end 94.36 102.5) (width 0.4) (layer F.Cu) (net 21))
 (segment (start 116.5 93.04) (end 103.82 93.04) (width 0.4) (layer F.Cu) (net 21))
 (segment (start 106.96 75) (end 110.5 78.54) (width 0.4) (layer F.Cu) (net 22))
 (segment (start 102.5 75) (end 106.96 75) (width 0.4) (layer F.Cu) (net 22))
 (segment (start 82.860001 86.059999) (end 81.66 87.26) (width 0.4) (layer F.Cu) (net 22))
 (segment (start 87.543999 86.059999) (end 82.860001 86.059999) (width 0.4) (layer F.Cu) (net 22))
 (segment (start 98.603998 75) (end 87.543999 86.059999) (width 0.4) (layer F.Cu) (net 22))
 (segment (start 102.5 75) (end 98.603998 75) (width 0.4) (layer F.Cu) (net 22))
 (segment (start 117.877999 94.202001) (end 114.797999 94.202001) (width 0.4) (layer F.Cu) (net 23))
 (segment (start 119.04 93.04) (end 117.877999 94.202001) (width 0.4) (layer F.Cu) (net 23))
 (segment (start 103.258009 96.141991) (end 96.9 102.5) (width 0.4) (layer F.Cu) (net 23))
 (segment (start 112.858009 96.141991) (end 103.258009 96.141991) (width 0.4) (layer F.Cu) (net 23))
 (segment (start 114.797999 94.202001) (end 112.858009 96.141991) (width 0.4) (layer F.Cu) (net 23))
 (segment (start 110.277999 96.742001) (end 104.52 102.5) (width 0.4) (layer F.Cu) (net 29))
 (segment (start 117.877999 96.742001) (end 110.277999 96.742001) (width 0.4) (layer F.Cu) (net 29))
 (segment (start 119.04 95.58) (end 117.877999 96.742001) (width 0.4) (layer F.Cu) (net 29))
 (segment (start 119.96 72.236839) (end 119.96 72.5) (width 0.4) (layer F.Cu) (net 2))
 (segment (start 120.846849 71.34999) (end 119.96 72.236839) (width 0.4) (layer F.Cu) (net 2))
 (segment (start 138.869923 71.34999) (end 120.846849 71.34999) (width 0.4) (layer F.Cu) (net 2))
 (segment (start 148 53.3) (end 148 62.219913) (width 0.4) (layer F.Cu) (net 2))
 (segment (start 40 102.5) (end 44 106.5) (width 0.4) (layer F.Cu) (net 2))
 (segment (start 44 106.5) (end 143 106.5) (width 0.4) (layer F.Cu) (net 2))
 (segment (start 143 106.5) (end 145 104.5) (width 0.4) (layer F.Cu) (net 2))
 (segment (start 145 65.219912) (end 145.109956 65.109956) (width 0.4) (layer F.Cu) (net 2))
 (segment (start 145 104.5) (end 145 65.219912) (width 0.4) (layer F.Cu) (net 2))
 (segment (start 145.109956 65.109956) (end 138.869923 71.34999) (width 0.4) (layer F.Cu) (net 2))
 (segment (start 148 62.219913) (end 145.109956 65.109956) (width 0.4) (layer F.Cu) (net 2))
 (segment (start 107.690798 102.5) (end 107.06 102.5) (width 0.4) (layer F.Cu) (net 30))
 (segment (start 112.070798 98.12) (end 107.690798 102.5) (width 0.4) (layer F.Cu) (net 30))
 (segment (start 116.5 98.12) (end 112.070798 98.12) (width 0.4) (layer F.Cu) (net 30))
 (segment (start 111.677999 91.877999) (end 107.06 87.26) (width 0.4) (layer F.Cu) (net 31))
 (segment (start 119.597761 91.877999) (end 111.677999 91.877999) (width 0.4) (layer F.Cu) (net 31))
 (segment (start 120.202001 92.482239) (end 119.597761 91.877999) (width 0.4) (layer F.Cu) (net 31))
 (segment (start 120.202001 93.597761) (end 120.202001 92.482239) (width 0.4) (layer F.Cu) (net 31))
 (segment (start 119.597761 94.202001) (end 120.202001 93.597761) (width 0.4) (layer F.Cu) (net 31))
 (segment (start 118.726541 94.202001) (end 119.597761 94.202001) (width 0.4) (layer F.Cu) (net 31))
 (segment (start 117.348542 95.58) (end 118.726541 94.202001) (width 0.4) (layer F.Cu) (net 31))
 (segment (start 116.5 95.58) (end 117.348542 95.58) (width 0.4) (layer F.Cu) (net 31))
 (segment (start 62.419999 90.419999) (end 63 91) (width 0.4) (layer F.Cu) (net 33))
 (segment (start 62.419999 75.580001) (end 62.419999 90.419999) (width 0.4) (layer F.Cu) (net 33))
 (segment (start 63.5 74.5) (end 62.419999 75.580001) (width 0.4) (layer F.Cu) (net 33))
 (segment (start 71.5 74.5) (end 72 74) (width 0.4) (layer F.Cu) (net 33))
 (segment (start 63.5 74.5) (end 71.5 74.5) (width 0.4) (layer F.Cu) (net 33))
 (segment (start 86.5 74) (end 87 74.5) (width 0.4) (layer F.Cu) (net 33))
 (segment (start 72 74) (end 86.5 74) (width 0.4) (layer F.Cu) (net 33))
 (segment (start 108.200001 73.700001) (end 110.5 76) (width 0.4) (layer F.Cu) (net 33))
 (segment (start 87.799999 73.700001) (end 108.200001 73.700001) (width 0.4) (layer F.Cu) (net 33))
 (segment (start 87 74.5) (end 87.799999 73.700001) (width 0.4) (layer F.Cu) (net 33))
 (segment (start 54 95.42) (end 53.58 95) (width 0.4) (layer F.Cu) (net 34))
 (segment (start 54 101.5) (end 54 95.42) (width 0.4) (layer F.Cu) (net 34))
 (segment (start 60.12 101.5) (end 63 98.62) (width 0.4) (layer F.Cu) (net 34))
 (segment (start 54 101.5) (end 60.12 101.5) (width 0.4) (layer F.Cu) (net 34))
 (segment (start 43.5 100.92) (end 45.08 102.5) (width 0.4) (layer F.Cu) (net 38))
 (segment (start 43.5 96) (end 43.5 100.92) (width 0.4) (layer F.Cu) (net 38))
 (segment (start 46.08 101.5) (end 45.08 102.5) (width 0.4) (layer F.Cu) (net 38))
 (segment (start 51 101.5) (end 46.08 101.5) (width 0.4) (layer F.Cu) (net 38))
 (segment (start 51 95.04) (end 51.04 95) (width 0.4) (layer F.Cu) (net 38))
 (segment (start 51 101.5) (end 51 95.04) (width 0.4) (layer F.Cu) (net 38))
 (segment (start 43.5 88.38) (end 43.5 91) (width 0.4) (layer F.Cu) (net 39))
 (segment (start 47.5 95) (end 48.5 95) (width 0.4) (layer F.Cu) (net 39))
 (segment (start 43.5 91) (end 47.5 95) (width 0.4) (layer F.Cu) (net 39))
 (segment (start 55.88 78.88) (end 56 79) (width 0.4) (layer F.Cu) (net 40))
 (segment (start 55.88 74.5) (end 55.88 78.88) (width 0.4) (layer F.Cu) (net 40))
 (segment (start 56 79.88) (end 56 79) (width 0.4) (layer F.Cu) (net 40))
 (segment (start 48.5 87.38) (end 56 79.88) (width 0.4) (layer F.Cu) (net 40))
 (segment (start 119.04 90.5) (end 119.04 84.96) (width 0.4) (layer F.Cu) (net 1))
 (segment (start 123 73) (end 122.5 72.5) (width 0.4) (layer F.Cu) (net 1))
 (segment (start 123 81) (end 123 73) (width 0.4) (layer F.Cu) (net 1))
 (segment (start 88.079999 86.683999) (end 89.763998 85) (width 0.4) (layer F.Cu) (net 1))
 (segment (start 88.079999 87.696003) (end 88.079999 86.683999) (width 0.4) (layer F.Cu) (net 1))
 (segment (start 87.316001 88.460001) (end 88.079999 87.696003) (width 0.4) (layer F.Cu) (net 1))
 (segment (start 72.700001 88.460001) (end 87.316001 88.460001) (width 0.4) (layer F.Cu) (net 1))
 (segment (start 71.5 87.26) (end 72.700001 88.460001) (width 0.4) (layer F.Cu) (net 1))
 (segment (start 119 85) (end 120.25 83.75) (width 0.4) (layer F.Cu) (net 1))
 (segment (start 89.763998 85) (end 119 85) (width 0.4) (layer F.Cu) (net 1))
 (segment (start 120.25 83.75) (end 123 81) (width 0.4) (layer F.Cu) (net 1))
 (segment (start 119.04 84.96) (end 120.25 83.75) (width 0.4) (layer F.Cu) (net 1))
 (segment (start 53.17 48.5) (end 42.67 59) (width 0.4) (layer F.Cu) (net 32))
 (segment (start 148 48.5) (end 53.17 48.5) (width 0.4) (layer F.Cu) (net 32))
 (segment (start 111.90001 79.67999) (end 110.5 81.08) (width 0.4) (layer F.Cu) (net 35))
 (segment (start 133.35002 70.74998) (end 120.176859 70.74998) (width 0.4) (layer F.Cu) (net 35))
 (segment (start 139 65.1) (end 133.35002 70.74998) (width 0.4) (layer F.Cu) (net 35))
 (segment (start 111.90001 79.026829) (end 111.90001 79.67999) (width 0.4) (layer F.Cu) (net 35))
 (segment (start 120.176859 70.74998) (end 111.90001 79.026829) (width 0.4) (layer F.Cu) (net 35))
 (segment (start 139 63.7) (end 139 65.1) (width 0.4) (layer F.Cu) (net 35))
 (segment (start 109.92 80.5) (end 110.5 81.08) (width 0.4) (layer F.Cu) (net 35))
 (segment (start 102.5 80.5) (end 109.92 80.5) (width 0.4) (layer F.Cu) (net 35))
 (segment (start 131.5 51.5) (end 130.5 50.5) (width 0.4) (layer F.Cu) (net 36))
 (segment (start 131.5 58.66) (end 131.5 51.5) (width 0.4) (layer F.Cu) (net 36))
 (segment (start 139 67.56) (end 139 68.74) (width 0.4) (layer B.Cu) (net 36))
 (segment (start 131.5 60.06) (end 139 67.56) (width 0.4) (layer B.Cu) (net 36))
 (segment (start 131.5 58.66) (end 131.5 60.06) (width 0.4) (layer B.Cu) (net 36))
 (segment (start 139 59.84) (end 139 58.66) (width 0.4) (layer F.Cu) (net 37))
 (segment (start 131.5 67.34) (end 139 59.84) (width 0.4) (layer F.Cu) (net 37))
 (segment (start 131.5 68.74) (end 131.5 67.34) (width 0.4) (layer F.Cu) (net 37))
 (segment (start 135.58 55.24) (end 139 58.66) (width 0.4) (layer F.Cu) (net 37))
 (segment (start 135.58 50.5) (end 135.58 55.24) (width 0.4) (layer F.Cu) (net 37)))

